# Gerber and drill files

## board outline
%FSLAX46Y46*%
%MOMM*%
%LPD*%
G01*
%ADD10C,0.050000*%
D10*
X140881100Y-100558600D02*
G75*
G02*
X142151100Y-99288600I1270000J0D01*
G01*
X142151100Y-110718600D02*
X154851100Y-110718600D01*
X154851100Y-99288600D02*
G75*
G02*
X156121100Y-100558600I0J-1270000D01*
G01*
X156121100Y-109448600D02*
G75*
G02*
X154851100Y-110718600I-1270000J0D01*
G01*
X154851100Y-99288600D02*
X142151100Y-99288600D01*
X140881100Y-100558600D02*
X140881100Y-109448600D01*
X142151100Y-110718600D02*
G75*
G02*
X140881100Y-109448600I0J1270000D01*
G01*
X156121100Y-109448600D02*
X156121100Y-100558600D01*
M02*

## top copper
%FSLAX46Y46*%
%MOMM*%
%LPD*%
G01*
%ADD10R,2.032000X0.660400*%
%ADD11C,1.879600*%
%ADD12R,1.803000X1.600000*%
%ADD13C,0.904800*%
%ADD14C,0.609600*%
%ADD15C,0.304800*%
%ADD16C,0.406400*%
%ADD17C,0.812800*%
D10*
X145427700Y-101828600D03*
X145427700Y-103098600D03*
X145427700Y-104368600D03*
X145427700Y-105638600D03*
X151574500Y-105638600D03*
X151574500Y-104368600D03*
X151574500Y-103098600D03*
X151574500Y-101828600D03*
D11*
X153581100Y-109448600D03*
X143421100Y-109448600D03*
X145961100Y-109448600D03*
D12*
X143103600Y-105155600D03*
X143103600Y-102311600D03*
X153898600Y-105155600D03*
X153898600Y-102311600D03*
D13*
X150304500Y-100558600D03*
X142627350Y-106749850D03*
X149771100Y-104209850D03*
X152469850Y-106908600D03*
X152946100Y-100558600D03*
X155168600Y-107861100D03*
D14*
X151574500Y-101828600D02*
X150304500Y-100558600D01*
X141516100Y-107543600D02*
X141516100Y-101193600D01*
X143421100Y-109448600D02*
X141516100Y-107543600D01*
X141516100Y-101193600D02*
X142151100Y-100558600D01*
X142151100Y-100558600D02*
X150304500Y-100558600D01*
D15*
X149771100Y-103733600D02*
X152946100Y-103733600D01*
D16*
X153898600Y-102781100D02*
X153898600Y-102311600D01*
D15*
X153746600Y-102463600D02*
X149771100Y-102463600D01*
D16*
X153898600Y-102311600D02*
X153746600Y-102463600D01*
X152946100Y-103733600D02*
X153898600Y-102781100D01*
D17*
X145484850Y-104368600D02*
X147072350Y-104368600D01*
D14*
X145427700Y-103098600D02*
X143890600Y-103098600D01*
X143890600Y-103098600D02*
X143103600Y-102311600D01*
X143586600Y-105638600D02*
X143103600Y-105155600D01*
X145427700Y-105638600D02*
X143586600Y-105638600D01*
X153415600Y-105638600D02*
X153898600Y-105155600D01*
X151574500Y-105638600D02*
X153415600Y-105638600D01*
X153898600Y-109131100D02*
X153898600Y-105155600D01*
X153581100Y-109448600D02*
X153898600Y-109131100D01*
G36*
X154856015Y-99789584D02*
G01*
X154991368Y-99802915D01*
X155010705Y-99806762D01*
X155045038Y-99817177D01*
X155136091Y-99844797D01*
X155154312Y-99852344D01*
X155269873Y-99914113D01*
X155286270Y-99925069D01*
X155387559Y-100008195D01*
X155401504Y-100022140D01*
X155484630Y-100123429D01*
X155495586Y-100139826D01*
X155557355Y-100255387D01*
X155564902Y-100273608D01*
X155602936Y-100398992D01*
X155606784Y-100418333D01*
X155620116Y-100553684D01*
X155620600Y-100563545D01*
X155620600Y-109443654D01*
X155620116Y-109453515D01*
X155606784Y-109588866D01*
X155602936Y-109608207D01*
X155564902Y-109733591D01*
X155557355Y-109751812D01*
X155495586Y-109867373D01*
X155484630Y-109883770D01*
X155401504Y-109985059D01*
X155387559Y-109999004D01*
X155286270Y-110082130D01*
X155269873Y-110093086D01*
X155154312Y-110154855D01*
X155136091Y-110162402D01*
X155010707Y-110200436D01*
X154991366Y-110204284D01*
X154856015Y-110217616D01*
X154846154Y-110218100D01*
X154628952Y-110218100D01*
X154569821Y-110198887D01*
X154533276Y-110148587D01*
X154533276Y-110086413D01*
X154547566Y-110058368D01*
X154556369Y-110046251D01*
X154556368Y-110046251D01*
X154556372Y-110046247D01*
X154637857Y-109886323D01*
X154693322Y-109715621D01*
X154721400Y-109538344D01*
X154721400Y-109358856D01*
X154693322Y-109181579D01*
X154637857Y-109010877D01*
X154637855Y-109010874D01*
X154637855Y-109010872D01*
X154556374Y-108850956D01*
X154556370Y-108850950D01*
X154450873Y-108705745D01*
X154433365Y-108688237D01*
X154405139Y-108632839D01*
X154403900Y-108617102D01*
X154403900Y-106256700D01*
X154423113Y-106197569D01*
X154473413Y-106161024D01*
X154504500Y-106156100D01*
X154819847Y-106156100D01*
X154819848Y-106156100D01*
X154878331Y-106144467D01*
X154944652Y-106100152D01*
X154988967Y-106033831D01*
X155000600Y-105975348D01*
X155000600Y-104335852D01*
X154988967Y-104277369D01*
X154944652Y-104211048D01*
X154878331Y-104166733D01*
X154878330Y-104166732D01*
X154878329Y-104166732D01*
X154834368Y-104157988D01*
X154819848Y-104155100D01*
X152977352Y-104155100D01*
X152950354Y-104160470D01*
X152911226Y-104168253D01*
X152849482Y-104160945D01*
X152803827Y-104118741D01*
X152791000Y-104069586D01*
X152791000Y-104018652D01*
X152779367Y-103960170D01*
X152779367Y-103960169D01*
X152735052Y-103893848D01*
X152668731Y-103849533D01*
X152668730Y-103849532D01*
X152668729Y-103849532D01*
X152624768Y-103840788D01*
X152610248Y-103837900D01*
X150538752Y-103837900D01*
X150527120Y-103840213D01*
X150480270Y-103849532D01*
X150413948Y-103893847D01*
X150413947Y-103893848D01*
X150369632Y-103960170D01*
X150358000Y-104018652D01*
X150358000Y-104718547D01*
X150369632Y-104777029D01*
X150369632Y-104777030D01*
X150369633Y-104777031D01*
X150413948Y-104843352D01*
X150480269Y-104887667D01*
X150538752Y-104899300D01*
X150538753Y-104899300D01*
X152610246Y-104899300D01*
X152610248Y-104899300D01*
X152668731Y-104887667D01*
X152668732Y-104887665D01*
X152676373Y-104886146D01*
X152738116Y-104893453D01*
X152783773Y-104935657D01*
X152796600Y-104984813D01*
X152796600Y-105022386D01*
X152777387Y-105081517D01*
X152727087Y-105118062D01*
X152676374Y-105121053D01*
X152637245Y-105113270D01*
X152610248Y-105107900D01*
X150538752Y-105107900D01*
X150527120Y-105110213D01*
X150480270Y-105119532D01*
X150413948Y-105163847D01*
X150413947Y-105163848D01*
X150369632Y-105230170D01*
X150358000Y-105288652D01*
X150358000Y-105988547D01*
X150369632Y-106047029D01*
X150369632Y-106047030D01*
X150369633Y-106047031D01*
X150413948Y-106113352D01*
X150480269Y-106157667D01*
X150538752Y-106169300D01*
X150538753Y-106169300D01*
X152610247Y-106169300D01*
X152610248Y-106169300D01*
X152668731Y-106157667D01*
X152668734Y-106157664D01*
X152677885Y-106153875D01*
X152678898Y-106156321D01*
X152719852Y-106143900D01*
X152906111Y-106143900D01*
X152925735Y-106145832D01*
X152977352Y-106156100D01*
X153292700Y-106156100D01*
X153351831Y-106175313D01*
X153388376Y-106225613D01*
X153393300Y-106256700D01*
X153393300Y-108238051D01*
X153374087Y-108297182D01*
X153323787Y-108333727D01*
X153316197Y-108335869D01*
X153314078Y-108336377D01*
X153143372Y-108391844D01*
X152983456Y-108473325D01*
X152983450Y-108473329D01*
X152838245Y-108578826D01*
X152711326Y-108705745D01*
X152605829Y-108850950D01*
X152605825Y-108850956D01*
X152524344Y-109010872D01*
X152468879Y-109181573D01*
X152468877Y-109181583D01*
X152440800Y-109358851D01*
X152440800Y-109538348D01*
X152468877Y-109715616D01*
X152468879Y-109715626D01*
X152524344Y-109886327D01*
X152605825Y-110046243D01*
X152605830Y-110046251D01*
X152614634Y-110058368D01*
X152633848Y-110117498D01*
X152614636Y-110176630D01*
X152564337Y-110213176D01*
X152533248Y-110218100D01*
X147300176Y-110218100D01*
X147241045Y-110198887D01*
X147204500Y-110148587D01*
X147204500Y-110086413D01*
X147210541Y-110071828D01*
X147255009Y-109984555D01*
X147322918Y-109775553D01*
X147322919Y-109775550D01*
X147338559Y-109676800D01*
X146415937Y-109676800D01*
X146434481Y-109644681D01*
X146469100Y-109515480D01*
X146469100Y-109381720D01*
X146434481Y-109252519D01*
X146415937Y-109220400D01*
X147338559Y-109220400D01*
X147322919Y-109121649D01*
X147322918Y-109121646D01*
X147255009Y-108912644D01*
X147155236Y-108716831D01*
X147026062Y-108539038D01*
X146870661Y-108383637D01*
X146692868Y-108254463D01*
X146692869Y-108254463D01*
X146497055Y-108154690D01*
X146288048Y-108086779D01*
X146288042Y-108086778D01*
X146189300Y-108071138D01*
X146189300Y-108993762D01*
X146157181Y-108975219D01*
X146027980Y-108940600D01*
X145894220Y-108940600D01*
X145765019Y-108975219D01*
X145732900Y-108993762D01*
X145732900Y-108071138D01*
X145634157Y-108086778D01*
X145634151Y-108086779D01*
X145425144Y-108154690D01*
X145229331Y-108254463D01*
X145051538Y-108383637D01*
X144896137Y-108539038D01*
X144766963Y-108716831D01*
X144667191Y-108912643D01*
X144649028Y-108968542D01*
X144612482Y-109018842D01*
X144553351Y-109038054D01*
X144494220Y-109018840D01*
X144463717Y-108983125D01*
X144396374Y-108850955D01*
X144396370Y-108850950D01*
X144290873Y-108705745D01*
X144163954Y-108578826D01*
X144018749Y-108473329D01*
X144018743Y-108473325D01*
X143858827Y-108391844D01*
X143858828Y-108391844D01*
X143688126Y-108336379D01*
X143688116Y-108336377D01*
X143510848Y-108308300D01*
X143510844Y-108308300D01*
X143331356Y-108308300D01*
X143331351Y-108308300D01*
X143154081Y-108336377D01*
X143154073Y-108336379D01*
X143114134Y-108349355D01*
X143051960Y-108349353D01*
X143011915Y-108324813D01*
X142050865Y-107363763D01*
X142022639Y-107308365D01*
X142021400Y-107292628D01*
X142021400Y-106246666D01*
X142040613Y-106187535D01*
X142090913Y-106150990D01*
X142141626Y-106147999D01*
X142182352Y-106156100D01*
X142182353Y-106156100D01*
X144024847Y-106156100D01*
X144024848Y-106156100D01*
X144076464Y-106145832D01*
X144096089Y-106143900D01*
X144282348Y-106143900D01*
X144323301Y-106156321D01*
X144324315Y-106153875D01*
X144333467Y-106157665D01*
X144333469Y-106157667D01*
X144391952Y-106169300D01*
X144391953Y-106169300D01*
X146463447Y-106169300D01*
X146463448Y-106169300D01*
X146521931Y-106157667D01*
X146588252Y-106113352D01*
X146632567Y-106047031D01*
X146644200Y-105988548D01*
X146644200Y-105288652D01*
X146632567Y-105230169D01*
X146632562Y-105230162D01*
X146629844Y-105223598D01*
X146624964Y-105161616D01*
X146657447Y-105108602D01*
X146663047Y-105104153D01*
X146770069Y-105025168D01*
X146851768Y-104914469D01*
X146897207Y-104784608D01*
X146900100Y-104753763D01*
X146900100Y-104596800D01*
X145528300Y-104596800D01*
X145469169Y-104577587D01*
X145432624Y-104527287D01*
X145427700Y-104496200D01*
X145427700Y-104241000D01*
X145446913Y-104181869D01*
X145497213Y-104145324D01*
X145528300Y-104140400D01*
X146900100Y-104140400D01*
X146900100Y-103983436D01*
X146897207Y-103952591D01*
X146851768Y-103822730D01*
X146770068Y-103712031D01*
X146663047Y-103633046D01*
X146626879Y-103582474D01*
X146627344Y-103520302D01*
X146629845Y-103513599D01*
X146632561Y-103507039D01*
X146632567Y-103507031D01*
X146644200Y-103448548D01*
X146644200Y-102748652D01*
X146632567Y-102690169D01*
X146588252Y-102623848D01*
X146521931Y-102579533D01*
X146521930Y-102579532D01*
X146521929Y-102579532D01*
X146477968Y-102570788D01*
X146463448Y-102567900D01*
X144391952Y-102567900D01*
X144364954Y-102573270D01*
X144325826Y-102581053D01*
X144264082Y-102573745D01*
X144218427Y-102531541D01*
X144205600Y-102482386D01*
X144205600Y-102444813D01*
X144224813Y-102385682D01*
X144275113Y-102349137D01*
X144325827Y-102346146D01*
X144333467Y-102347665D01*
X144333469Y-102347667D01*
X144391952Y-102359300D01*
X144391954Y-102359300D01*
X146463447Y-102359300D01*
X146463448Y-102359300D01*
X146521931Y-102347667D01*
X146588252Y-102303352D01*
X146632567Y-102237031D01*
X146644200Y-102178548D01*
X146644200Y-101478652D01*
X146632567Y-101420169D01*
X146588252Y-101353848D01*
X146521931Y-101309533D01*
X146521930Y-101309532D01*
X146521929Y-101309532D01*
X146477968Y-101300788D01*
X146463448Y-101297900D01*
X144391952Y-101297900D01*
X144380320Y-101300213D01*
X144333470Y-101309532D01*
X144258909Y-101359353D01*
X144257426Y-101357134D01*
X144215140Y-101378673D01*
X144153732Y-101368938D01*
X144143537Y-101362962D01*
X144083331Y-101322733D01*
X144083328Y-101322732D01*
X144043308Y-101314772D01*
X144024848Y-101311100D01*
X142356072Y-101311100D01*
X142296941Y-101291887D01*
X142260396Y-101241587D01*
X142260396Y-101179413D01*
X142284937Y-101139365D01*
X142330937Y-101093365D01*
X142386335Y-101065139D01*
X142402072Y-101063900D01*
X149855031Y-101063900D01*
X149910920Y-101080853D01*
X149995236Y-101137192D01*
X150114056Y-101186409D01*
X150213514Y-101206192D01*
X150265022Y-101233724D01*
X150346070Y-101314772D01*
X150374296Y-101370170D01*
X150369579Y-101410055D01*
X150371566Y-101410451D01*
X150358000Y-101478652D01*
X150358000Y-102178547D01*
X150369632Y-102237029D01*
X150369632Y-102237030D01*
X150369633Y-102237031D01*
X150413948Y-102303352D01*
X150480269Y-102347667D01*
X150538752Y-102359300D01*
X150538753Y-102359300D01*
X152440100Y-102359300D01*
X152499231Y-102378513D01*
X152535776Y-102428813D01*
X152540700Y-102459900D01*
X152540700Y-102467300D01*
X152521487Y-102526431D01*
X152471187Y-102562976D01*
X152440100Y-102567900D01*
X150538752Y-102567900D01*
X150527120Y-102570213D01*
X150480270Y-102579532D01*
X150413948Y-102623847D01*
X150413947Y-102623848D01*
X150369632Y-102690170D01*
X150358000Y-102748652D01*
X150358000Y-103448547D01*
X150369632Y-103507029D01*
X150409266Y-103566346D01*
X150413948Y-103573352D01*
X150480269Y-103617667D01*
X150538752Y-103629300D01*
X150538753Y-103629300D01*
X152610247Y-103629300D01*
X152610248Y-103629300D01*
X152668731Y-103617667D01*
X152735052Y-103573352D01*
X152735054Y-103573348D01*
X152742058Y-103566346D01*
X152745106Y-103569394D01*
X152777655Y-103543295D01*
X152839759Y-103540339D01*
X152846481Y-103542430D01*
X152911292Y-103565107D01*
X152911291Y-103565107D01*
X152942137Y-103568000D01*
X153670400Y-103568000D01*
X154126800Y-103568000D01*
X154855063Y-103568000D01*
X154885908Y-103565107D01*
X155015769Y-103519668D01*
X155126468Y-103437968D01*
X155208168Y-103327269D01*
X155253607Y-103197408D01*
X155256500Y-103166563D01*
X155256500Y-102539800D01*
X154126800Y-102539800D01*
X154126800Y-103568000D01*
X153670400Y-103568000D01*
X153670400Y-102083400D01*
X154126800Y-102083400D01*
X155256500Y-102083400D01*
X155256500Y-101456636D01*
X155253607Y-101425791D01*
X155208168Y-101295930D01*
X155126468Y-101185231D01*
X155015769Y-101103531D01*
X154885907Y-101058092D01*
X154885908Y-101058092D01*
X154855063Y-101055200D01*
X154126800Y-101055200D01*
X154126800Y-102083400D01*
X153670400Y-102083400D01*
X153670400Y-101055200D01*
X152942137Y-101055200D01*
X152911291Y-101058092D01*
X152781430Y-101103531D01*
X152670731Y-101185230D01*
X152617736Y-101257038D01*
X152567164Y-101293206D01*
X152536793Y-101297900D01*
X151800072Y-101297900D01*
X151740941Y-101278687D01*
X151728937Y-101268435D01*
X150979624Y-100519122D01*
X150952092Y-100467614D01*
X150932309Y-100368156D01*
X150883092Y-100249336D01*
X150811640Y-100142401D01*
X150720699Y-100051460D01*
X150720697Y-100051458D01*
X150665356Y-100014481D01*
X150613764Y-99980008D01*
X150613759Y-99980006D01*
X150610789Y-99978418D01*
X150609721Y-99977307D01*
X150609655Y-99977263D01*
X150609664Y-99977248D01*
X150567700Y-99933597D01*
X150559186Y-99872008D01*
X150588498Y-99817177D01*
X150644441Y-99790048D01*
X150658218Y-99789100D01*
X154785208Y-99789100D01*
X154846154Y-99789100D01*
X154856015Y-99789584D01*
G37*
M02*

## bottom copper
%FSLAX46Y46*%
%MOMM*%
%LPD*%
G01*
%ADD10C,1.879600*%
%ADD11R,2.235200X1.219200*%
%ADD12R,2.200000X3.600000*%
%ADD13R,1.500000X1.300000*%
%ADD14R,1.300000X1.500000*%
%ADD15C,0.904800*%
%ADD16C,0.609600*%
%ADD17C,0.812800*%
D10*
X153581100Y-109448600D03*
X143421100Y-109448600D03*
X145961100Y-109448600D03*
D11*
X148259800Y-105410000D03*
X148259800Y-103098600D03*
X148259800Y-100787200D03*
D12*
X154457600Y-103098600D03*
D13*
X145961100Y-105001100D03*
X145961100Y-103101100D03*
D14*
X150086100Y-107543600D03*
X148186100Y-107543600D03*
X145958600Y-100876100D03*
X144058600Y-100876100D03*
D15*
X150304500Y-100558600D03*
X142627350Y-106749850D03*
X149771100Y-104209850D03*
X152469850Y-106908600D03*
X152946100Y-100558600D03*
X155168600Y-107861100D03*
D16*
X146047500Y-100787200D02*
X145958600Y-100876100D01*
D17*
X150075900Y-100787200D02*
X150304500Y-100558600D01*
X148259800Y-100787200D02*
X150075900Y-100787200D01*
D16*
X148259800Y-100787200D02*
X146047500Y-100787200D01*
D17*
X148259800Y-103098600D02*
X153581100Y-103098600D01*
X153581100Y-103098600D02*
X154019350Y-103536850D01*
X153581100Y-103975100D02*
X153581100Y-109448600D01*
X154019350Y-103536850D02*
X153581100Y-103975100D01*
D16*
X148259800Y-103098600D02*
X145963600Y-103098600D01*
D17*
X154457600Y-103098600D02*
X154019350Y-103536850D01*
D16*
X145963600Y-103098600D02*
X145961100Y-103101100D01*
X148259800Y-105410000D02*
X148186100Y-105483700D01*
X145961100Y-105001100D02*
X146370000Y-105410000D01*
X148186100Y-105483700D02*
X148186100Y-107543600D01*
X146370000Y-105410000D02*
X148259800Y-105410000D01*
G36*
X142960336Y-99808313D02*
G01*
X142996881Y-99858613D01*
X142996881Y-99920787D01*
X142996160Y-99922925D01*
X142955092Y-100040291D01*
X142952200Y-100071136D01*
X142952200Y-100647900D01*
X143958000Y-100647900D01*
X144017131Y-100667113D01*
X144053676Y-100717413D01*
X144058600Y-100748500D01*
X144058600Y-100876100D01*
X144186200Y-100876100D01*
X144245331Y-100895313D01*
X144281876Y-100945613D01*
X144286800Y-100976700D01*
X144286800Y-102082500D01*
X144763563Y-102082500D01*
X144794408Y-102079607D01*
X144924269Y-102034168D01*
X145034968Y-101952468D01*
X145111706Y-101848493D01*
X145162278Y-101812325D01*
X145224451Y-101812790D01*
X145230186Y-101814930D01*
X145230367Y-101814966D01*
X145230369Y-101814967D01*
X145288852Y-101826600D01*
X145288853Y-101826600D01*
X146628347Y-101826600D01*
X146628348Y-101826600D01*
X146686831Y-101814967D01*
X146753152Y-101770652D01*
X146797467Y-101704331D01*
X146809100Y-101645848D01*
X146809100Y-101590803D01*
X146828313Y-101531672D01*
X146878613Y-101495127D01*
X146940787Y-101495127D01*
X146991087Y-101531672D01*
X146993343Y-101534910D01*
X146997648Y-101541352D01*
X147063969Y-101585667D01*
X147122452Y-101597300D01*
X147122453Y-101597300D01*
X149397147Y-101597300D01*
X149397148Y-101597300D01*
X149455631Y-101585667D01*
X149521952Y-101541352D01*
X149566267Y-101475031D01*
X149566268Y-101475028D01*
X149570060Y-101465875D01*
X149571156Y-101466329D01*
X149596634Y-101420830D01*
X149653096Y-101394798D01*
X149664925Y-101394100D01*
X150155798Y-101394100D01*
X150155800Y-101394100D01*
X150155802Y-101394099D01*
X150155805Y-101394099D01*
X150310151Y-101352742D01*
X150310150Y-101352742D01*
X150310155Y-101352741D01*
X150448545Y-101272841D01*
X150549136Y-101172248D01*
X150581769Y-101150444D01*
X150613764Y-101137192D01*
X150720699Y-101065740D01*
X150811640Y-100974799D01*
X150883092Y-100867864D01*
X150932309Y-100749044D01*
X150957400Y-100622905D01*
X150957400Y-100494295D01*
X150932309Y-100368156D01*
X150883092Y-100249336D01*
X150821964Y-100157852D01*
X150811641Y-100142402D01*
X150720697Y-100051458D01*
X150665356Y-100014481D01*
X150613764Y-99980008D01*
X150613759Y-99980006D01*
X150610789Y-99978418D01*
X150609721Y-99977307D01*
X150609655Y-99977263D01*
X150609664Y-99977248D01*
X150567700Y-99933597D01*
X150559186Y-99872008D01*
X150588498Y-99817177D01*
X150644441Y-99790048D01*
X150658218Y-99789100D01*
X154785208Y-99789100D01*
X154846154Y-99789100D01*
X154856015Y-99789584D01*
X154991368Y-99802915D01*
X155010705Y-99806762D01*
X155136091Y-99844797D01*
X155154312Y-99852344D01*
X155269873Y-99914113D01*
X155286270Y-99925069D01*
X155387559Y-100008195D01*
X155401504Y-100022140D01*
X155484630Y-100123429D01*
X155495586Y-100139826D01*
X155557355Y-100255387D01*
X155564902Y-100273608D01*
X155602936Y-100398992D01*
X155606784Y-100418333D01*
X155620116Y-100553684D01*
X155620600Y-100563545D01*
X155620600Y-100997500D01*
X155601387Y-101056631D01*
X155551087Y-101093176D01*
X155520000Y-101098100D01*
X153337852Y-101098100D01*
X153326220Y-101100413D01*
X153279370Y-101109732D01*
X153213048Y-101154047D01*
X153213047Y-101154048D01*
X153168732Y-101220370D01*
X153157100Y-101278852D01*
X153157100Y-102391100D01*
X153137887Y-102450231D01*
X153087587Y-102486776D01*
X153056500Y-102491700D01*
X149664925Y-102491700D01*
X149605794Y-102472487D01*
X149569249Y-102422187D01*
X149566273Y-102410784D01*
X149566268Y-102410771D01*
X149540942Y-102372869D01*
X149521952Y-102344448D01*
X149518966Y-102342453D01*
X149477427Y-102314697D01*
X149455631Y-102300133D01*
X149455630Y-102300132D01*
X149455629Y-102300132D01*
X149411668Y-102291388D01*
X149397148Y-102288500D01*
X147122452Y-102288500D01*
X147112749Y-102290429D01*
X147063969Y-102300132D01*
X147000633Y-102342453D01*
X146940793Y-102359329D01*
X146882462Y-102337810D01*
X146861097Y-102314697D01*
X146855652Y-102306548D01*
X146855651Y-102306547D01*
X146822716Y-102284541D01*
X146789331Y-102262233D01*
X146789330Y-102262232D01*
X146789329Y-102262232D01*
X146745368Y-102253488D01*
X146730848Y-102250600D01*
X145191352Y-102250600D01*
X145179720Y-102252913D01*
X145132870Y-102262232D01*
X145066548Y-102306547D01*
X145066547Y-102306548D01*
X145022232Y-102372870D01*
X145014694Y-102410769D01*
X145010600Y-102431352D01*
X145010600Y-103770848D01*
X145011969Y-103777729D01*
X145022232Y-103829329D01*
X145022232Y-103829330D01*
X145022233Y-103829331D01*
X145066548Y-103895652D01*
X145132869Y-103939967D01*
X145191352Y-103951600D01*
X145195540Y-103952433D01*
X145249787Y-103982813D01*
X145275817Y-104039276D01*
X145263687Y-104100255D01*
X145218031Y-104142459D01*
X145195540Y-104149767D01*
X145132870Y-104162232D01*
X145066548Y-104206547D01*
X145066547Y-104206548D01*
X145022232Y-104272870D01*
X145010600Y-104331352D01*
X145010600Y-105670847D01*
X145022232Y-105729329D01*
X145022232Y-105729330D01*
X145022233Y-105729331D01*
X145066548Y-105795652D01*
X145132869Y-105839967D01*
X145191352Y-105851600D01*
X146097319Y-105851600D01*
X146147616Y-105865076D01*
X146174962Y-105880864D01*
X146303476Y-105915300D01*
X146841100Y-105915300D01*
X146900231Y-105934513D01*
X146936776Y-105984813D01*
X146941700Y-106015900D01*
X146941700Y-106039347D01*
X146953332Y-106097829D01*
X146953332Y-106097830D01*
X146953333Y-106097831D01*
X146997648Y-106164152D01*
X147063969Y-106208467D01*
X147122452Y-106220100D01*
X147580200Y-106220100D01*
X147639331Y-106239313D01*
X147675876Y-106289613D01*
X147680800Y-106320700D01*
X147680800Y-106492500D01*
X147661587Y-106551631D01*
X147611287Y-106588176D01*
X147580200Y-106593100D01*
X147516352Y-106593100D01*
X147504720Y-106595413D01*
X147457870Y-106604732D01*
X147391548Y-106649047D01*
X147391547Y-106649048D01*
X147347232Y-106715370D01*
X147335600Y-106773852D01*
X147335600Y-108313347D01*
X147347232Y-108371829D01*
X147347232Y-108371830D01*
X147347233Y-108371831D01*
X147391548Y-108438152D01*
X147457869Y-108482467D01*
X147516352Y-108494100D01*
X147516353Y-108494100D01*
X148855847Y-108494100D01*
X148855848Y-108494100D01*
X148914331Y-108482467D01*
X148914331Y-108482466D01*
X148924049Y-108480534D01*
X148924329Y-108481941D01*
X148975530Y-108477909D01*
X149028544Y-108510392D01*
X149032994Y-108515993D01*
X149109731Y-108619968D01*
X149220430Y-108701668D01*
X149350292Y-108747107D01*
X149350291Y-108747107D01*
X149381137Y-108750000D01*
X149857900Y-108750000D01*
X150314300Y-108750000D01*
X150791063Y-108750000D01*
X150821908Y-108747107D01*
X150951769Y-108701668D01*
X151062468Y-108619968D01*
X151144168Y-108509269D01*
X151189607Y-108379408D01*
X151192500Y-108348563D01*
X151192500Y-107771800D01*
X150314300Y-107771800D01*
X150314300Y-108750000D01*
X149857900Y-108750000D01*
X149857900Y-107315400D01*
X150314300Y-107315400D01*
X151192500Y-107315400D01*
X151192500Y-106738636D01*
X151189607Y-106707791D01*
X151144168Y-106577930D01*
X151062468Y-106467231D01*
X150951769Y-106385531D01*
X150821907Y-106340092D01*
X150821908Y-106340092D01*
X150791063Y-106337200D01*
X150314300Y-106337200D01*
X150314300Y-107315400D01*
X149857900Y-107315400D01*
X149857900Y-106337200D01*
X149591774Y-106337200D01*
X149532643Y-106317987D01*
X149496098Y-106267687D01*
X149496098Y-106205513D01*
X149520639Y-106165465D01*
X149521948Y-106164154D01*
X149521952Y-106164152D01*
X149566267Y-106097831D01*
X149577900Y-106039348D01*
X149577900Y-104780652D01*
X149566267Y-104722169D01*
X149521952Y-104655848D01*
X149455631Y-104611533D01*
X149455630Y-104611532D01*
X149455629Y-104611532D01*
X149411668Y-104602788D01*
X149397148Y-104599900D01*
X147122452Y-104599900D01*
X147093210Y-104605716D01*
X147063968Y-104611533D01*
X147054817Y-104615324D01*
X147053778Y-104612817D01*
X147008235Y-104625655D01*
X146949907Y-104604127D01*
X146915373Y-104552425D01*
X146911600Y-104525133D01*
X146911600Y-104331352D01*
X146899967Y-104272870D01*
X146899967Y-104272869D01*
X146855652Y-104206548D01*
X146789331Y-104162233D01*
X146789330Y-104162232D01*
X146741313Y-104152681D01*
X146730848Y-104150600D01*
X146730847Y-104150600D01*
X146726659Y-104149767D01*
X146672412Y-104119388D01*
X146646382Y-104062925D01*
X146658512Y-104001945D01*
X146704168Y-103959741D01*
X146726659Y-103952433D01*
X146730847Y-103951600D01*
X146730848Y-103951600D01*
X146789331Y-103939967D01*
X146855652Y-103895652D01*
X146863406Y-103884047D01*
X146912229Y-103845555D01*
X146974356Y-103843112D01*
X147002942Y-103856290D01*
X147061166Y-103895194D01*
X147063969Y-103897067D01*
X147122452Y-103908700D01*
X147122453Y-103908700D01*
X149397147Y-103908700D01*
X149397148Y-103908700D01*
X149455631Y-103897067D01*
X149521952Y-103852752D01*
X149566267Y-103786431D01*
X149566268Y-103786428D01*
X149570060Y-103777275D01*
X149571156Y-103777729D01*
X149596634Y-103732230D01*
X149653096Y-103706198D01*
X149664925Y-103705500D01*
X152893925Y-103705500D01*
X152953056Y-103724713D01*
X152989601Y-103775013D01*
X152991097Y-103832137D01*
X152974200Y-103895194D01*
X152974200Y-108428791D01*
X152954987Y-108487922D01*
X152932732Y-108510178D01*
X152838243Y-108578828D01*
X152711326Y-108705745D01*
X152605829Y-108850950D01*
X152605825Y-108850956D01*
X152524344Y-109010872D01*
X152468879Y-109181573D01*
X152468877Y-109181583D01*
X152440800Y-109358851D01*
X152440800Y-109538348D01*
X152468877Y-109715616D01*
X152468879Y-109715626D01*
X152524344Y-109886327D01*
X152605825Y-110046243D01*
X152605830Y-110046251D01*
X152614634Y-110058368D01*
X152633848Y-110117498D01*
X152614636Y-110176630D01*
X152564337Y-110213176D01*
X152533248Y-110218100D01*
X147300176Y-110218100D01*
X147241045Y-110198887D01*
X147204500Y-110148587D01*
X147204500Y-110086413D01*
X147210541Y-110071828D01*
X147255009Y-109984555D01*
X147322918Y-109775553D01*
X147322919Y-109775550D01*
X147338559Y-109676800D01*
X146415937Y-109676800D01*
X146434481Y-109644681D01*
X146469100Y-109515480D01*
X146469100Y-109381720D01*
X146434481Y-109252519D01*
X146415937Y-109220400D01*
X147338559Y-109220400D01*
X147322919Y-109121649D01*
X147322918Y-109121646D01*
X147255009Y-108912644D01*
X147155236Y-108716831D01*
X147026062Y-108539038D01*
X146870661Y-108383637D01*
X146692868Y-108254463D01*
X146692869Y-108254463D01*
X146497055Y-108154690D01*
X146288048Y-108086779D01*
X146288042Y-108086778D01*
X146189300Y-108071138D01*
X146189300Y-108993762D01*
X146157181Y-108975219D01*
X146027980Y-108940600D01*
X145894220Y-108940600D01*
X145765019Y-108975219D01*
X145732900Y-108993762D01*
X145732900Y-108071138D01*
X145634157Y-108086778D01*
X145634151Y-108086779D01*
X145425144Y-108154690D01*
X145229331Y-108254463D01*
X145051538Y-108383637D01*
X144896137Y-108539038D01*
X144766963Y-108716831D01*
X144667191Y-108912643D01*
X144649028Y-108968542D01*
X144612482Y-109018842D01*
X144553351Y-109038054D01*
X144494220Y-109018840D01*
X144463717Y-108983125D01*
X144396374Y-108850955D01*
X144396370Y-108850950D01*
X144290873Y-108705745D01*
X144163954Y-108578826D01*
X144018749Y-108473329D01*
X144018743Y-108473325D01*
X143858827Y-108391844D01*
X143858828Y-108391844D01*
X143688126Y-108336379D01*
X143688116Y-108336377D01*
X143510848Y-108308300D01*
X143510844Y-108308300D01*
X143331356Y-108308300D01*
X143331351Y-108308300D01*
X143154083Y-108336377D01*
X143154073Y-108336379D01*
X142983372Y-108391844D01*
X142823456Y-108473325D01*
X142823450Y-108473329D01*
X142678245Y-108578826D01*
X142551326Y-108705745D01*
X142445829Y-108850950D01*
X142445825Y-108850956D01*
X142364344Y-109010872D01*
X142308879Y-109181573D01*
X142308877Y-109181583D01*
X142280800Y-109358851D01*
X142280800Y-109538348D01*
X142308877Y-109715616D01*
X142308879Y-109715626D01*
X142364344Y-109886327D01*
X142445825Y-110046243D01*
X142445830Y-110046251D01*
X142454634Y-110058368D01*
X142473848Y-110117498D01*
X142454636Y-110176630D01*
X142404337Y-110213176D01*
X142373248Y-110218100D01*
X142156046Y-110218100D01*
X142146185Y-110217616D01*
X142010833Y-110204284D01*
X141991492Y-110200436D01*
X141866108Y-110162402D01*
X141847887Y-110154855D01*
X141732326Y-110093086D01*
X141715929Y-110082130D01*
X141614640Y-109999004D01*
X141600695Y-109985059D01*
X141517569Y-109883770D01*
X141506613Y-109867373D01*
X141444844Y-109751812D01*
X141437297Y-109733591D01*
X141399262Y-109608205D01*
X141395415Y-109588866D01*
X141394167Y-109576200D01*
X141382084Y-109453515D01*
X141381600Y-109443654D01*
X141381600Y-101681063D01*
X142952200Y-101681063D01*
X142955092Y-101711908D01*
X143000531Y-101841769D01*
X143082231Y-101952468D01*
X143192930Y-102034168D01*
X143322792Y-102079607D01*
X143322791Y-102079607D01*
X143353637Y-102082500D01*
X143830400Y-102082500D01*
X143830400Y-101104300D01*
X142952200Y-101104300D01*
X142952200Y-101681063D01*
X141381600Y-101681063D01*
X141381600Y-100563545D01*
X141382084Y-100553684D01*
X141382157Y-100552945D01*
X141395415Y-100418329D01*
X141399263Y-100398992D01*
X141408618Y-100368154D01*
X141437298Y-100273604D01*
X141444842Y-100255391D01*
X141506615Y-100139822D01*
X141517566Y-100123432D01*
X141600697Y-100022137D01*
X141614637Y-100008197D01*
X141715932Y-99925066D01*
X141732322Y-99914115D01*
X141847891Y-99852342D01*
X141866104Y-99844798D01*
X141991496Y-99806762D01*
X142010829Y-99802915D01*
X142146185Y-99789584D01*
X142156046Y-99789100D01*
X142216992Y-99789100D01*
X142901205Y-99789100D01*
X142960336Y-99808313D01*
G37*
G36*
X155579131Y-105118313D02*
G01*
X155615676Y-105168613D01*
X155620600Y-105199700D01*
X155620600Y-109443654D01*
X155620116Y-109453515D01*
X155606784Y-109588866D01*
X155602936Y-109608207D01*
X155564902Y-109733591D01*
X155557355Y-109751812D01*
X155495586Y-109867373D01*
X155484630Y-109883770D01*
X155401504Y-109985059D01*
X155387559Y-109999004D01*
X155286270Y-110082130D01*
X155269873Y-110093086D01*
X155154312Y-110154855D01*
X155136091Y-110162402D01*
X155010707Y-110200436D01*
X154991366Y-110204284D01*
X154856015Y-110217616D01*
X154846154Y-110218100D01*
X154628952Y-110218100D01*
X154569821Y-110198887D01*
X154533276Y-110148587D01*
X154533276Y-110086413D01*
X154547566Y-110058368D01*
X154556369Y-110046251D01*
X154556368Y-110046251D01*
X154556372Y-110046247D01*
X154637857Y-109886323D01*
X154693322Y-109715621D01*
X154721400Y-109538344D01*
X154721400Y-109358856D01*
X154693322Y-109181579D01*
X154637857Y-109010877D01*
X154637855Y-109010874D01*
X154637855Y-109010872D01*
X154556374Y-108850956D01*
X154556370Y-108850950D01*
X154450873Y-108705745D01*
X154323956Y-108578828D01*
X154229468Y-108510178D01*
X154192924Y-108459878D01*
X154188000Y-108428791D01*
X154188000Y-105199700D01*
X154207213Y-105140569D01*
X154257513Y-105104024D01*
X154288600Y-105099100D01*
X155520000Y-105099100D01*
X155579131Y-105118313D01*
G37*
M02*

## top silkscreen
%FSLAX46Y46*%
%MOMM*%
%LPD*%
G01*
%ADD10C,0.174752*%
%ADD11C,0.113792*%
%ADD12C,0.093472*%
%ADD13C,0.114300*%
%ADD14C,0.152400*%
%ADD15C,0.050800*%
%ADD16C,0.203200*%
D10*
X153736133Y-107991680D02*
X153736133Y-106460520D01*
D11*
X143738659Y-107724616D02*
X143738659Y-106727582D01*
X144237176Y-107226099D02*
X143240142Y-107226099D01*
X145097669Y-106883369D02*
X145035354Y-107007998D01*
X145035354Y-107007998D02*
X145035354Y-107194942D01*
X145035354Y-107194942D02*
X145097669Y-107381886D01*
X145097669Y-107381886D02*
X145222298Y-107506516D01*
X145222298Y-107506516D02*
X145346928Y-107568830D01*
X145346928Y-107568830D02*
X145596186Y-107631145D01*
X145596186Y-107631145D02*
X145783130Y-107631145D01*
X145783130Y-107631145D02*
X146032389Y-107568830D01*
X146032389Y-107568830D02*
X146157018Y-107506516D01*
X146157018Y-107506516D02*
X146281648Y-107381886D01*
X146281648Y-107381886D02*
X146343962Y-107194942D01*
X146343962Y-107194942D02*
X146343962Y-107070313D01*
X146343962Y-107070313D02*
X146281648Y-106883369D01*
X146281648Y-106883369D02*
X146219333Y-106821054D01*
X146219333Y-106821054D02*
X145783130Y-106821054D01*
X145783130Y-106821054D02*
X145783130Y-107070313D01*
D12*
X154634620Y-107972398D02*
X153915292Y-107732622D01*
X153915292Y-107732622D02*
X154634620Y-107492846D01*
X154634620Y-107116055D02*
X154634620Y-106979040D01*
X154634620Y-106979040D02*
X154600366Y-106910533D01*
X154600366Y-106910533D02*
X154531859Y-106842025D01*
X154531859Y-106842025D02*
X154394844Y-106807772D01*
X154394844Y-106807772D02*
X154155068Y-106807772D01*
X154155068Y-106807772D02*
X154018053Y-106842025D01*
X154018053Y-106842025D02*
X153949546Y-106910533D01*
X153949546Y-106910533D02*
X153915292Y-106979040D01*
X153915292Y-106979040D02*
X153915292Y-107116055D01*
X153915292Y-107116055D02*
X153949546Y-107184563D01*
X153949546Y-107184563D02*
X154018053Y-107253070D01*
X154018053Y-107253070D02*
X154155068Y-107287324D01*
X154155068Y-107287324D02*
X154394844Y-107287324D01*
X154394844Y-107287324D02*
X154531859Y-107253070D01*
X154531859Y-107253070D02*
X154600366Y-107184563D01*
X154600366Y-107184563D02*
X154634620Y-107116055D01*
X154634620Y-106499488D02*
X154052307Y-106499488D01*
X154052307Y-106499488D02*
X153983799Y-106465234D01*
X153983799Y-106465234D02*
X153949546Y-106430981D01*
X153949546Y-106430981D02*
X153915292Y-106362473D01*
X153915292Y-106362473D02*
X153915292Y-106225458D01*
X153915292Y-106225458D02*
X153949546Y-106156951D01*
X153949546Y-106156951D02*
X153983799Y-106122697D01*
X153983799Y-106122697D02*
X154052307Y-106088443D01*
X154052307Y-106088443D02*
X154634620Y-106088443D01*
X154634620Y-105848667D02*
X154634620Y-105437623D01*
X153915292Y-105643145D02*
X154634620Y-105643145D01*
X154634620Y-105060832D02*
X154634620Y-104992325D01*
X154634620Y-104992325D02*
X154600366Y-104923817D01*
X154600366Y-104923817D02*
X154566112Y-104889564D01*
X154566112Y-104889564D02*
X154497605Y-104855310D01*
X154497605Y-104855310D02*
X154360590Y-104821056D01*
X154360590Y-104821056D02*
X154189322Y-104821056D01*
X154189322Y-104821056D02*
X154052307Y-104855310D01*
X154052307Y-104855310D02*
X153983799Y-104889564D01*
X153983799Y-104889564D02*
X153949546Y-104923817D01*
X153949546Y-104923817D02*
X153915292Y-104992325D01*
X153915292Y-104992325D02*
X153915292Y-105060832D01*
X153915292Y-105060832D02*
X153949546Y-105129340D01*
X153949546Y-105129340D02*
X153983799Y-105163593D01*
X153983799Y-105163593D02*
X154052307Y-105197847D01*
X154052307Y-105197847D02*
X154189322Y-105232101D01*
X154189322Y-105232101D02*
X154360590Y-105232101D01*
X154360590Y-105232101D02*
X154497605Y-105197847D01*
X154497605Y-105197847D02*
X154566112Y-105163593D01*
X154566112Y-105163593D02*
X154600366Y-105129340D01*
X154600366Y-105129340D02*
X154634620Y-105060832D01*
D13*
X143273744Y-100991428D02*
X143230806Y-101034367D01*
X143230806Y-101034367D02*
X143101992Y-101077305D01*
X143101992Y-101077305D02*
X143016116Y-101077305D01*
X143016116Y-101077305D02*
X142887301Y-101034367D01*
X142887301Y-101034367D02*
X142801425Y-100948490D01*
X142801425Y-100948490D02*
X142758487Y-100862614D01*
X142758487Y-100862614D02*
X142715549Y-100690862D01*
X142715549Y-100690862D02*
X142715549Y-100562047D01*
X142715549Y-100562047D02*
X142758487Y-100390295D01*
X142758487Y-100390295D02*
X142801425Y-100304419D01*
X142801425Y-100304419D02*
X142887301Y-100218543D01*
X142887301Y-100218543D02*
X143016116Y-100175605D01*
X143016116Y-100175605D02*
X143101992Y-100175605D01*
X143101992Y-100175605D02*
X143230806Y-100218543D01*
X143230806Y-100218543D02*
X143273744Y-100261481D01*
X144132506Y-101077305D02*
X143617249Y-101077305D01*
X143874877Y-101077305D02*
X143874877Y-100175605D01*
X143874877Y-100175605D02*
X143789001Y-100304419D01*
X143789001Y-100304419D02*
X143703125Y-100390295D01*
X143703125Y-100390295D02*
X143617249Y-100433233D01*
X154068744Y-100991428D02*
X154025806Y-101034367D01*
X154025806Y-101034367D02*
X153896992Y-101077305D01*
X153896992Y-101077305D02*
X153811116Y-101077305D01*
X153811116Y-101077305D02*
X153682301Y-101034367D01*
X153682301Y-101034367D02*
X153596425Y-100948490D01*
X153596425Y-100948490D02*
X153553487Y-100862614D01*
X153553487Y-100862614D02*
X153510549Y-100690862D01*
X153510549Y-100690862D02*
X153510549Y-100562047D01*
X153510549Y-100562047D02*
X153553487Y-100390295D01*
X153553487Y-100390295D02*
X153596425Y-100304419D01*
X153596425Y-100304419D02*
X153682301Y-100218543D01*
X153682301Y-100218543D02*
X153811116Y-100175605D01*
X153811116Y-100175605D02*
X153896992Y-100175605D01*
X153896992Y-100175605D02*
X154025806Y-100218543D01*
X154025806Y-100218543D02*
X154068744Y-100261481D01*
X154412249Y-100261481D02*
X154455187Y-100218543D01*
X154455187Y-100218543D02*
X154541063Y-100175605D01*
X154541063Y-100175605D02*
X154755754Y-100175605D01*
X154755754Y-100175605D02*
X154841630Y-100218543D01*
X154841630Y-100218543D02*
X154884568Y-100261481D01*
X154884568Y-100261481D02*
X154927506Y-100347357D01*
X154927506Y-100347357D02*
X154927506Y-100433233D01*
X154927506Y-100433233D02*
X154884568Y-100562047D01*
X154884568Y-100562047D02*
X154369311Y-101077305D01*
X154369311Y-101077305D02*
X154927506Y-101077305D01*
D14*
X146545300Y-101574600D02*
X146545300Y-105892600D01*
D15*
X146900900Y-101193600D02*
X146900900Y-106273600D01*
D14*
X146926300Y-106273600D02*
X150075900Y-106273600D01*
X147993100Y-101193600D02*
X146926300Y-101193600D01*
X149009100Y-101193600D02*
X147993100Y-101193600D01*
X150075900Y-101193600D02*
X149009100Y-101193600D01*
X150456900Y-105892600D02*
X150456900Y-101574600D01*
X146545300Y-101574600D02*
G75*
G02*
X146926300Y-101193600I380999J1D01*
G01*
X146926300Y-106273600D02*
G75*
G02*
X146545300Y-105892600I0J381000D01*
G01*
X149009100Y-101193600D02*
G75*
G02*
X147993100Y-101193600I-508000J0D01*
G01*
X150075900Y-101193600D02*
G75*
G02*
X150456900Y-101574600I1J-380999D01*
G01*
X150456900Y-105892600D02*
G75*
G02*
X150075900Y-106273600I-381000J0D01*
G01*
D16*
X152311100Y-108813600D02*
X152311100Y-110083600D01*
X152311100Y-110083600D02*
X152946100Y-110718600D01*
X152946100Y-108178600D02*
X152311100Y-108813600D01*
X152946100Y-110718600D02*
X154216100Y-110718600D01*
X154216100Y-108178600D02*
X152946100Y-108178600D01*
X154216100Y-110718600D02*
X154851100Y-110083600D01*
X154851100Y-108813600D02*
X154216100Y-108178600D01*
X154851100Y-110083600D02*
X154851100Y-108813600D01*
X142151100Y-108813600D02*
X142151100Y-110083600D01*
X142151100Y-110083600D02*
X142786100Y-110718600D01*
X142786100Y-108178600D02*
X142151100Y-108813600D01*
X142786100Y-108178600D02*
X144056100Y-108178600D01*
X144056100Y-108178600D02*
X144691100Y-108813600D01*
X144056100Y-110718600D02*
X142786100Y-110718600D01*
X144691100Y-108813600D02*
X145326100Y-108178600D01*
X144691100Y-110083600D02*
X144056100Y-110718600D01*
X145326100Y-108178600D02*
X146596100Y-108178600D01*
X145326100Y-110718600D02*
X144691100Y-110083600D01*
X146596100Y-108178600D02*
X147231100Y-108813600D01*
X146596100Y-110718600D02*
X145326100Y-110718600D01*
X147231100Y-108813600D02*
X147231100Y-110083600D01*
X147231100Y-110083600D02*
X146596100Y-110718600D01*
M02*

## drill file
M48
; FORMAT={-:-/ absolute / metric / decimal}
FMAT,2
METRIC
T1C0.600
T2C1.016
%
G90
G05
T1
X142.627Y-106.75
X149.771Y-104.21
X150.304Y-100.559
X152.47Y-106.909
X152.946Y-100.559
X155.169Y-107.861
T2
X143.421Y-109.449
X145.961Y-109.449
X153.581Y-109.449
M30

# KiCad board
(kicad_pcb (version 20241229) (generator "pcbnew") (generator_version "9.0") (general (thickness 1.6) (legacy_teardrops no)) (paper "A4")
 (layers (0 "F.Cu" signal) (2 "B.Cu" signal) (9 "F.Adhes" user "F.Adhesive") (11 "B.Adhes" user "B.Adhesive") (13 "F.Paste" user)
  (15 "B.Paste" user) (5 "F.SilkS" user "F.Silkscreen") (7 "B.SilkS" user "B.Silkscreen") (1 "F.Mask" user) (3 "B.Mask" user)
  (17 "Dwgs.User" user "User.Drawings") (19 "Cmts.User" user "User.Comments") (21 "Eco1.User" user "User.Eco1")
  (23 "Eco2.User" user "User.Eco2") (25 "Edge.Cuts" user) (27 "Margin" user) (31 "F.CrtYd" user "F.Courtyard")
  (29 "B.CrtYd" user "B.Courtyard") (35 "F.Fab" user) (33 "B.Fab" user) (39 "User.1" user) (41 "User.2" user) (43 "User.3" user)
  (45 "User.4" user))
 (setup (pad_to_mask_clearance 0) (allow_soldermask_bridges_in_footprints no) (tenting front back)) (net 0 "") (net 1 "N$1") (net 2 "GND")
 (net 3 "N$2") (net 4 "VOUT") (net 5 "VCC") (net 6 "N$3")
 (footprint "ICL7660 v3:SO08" (layer "F.Cu") (at 148.5011 103.7336 -90)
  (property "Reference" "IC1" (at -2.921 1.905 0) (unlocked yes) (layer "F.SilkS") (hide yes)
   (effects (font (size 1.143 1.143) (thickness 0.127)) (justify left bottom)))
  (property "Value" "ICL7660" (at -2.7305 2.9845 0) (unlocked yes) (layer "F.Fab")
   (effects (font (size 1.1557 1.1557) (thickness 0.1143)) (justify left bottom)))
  (fp_line (start -2.159 1.9558) (end 2.159 1.9558) (stroke (width 0.1524) (type solid)) (layer "F.SilkS"))
  (fp_line (start -2.54 1.6002) (end 2.54 1.6002) (stroke (width 0.0508) (type solid)) (layer "F.SilkS"))
  (fp_line (start 2.54 1.5748) (end 2.54 -1.5748) (stroke (width 0.1524) (type solid)) (layer "F.SilkS"))
  (fp_line (start -2.54 0.508) (end -2.54 1.5748) (stroke (width 0.1524) (type solid)) (layer "F.SilkS"))
  (fp_line (start -2.54 -0.508) (end -2.54 0.508) (stroke (width 0.1524) (type solid)) (layer "F.SilkS"))
  (fp_line (start -2.54 -1.5748) (end -2.54 -0.508) (stroke (width 0.1524) (type solid)) (layer "F.SilkS"))
  (fp_line (start 2.159 -1.9558) (end -2.159 -1.9558) (stroke (width 0.1524) (type solid)) (layer "F.SilkS"))
  (fp_arc (start -2.159 1.9558) (mid -2.428408 1.844208) (end -2.54 1.5748) (stroke (width 0.1524) (type solid)) (layer "F.SilkS"))
  (fp_arc (start 2.54 1.5748) (mid 2.428408 1.844208) (end 2.159 1.9558) (stroke (width 0.1524) (type solid)) (layer "F.SilkS"))
  (fp_arc (start -2.54 -0.508) (mid -2.032 0) (end -2.54 0.508) (stroke (width 0.1524) (type solid)) (layer "F.SilkS"))
  (fp_arc (start -2.54 -1.5748) (mid -2.428408 -1.844208) (end -2.159 -1.9558) (stroke (width 0.1524) (type solid)) (layer "F.SilkS"))
  (fp_arc (start 2.159 -1.9558) (mid 2.428408 -1.844208) (end 2.54 -1.5748) (stroke (width 0.1524) (type solid)) (layer "F.SilkS"))
  (pad "1" smd rect (at -1.905 3.0734 270) (size 0.6604 2.032) (layers "F.Cu" "F.Mask" "F.Paste") (solder_mask_margin 0.0508)
   (solder_paste_margin 0) (thermal_bridge_angle 0))
  (pad "2" smd rect (at -0.635 3.0734 270) (size 0.6604 2.032) (layers "F.Cu" "F.Mask" "F.Paste") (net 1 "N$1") (solder_mask_margin 0.0508)
   (solder_paste_margin 0) (thermal_bridge_angle 0))
  (pad "3" smd rect (at 0.635 3.0734 270) (size 0.6604 2.032) (layers "F.Cu" "F.Mask" "F.Paste") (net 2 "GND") (solder_mask_margin 0.0508)
   (solder_paste_margin 0) (thermal_bridge_angle 0))
  (pad "4" smd rect (at 1.905 3.0734 270) (size 0.6604 2.032) (layers "F.Cu" "F.Mask" "F.Paste") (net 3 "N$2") (solder_mask_margin 0.0508)
   (solder_paste_margin 0) (thermal_bridge_angle 0))
  (pad "5" smd rect (at 1.905 -3.0734 270) (size 0.6604 2.032) (layers "F.Cu" "F.Mask" "F.Paste") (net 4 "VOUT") (solder_mask_margin 0.0508)
   (solder_paste_margin 0) (thermal_bridge_angle 0))
  (pad "6" smd rect (at 0.635 -3.0734 270) (size 0.6604 2.032) (layers "F.Cu" "F.Mask" "F.Paste") (solder_mask_margin 0.0508)
   (solder_paste_margin 0) (thermal_bridge_angle 0))
  (pad "7" smd rect (at -0.635 -3.0734 270) (size 0.6604 2.032) (layers "F.Cu" "F.Mask" "F.Paste") (solder_mask_margin 0.0508)
   (solder_paste_margin 0) (thermal_bridge_angle 0))
  (pad "8" smd rect (at -1.905 -3.0734 270) (size 0.6604 2.032) (layers "F.Cu" "F.Mask" "F.Paste") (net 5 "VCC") (solder_mask_margin 0.0508)
   (solder_paste_margin 0) (thermal_bridge_angle 0)))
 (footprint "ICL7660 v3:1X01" (layer "F.Cu") (at 153.5811 109.4486)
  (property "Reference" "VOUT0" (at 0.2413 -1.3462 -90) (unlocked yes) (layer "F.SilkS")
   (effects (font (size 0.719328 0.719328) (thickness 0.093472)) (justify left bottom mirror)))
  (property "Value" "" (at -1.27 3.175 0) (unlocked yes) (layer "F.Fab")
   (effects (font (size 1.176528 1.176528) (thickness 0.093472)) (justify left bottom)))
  (fp_line (start -1.27 -0.635) (end -1.27 0.635) (stroke (width 0.2032) (type solid)) (layer "F.SilkS"))
  (fp_line (start -1.27 0.635) (end -0.635 1.27) (stroke (width 0.2032) (type solid)) (layer "F.SilkS"))
  (fp_line (start -0.635 -1.27) (end -1.27 -0.635) (stroke (width 0.2032) (type solid)) (layer "F.SilkS"))
  (fp_line (start -0.635 1.27) (end 0.635 1.27) (stroke (width 0.2032) (type solid)) (layer "F.SilkS"))
  (fp_line (start 0.635 -1.27) (end -0.635 -1.27) (stroke (width 0.2032) (type solid)) (layer "F.SilkS"))
  (fp_line (start 0.635 1.27) (end 1.27 0.635) (stroke (width 0.2032) (type solid)) (layer "F.SilkS"))
  (fp_line (start 1.27 -0.635) (end 0.635 -1.27) (stroke (width 0.2032) (type solid)) (layer "F.SilkS"))
  (fp_line (start 1.27 0.635) (end 1.27 -0.635) (stroke (width 0.2032) (type solid)) (layer "F.SilkS"))
  (pad "1" thru_hole circle (at 0 0 90) (size 1.8796 1.8796) (drill 1.016) (layers "*.Cu" "*.Mask") (remove_unused_layers no) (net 4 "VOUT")
   (solder_mask_margin 0.0508) (thermal_bridge_angle 0)))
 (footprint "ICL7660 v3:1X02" (layer "F.Cu") (at 143.4211 109.4486)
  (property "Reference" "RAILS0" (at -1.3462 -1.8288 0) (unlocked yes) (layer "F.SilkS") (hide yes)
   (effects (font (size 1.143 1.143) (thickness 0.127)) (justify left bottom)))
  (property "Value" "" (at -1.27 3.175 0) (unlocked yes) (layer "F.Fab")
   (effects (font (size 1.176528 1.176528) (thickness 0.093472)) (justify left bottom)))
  (fp_line (start -1.27 -0.635) (end -1.27 0.635) (stroke (width 0.2032) (type solid)) (layer "F.SilkS"))
  (fp_line (start -1.27 0.635) (end -0.635 1.27) (stroke (width 0.2032) (type solid)) (layer "F.SilkS"))
  (fp_line (start -0.635 -1.27) (end -1.27 -0.635) (stroke (width 0.2032) (type solid)) (layer "F.SilkS"))
  (fp_line (start -0.635 -1.27) (end 0.635 -1.27) (stroke (width 0.2032) (type solid)) (layer "F.SilkS"))
  (fp_line (start 0.635 -1.27) (end 1.27 -0.635) (stroke (width 0.2032) (type solid)) (layer "F.SilkS"))
  (fp_line (start 0.635 1.27) (end -0.635 1.27) (stroke (width 0.2032) (type solid)) (layer "F.SilkS"))
  (fp_line (start 1.27 -0.635) (end 1.905 -1.27) (stroke (width 0.2032) (type solid)) (layer "F.SilkS"))
  (fp_line (start 1.27 0.635) (end 0.635 1.27) (stroke (width 0.2032) (type solid)) (layer "F.SilkS"))
  (fp_line (start 1.905 -1.27) (end 3.175 -1.27) (stroke (width 0.2032) (type solid)) (layer "F.SilkS"))
  (fp_line (start 1.905 1.27) (end 1.27 0.635) (stroke (width 0.2032) (type solid)) (layer "F.SilkS"))
  (fp_line (start 3.175 -1.27) (end 3.81 -0.635) (stroke (width 0.2032) (type solid)) (layer "F.SilkS"))
  (fp_line (start 3.175 1.27) (end 1.905 1.27) (stroke (width 0.2032) (type solid)) (layer "F.SilkS"))
  (fp_line (start 3.81 -0.635) (end 3.81 0.635) (stroke (width 0.2032) (type solid)) (layer "F.SilkS"))
  (fp_line (start 3.81 0.635) (end 3.175 1.27) (stroke (width 0.2032) (type solid)) (layer "F.SilkS"))
  (pad "1" thru_hole circle (at 0 0 90) (size 1.8796 1.8796) (drill 1.016) (layers "*.Cu" "*.Mask") (remove_unused_layers no) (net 5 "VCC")
   (solder_mask_margin 0.0508) (thermal_bridge_angle 0))
  (pad "2" thru_hole circle (at 2.54 0 90) (size 1.8796 1.8796) (drill 1.016) (layers "*.Cu" "*.Mask") (remove_unused_layers no)
   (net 2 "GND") (solder_mask_margin 0.0508) (thermal_bridge_angle 0)))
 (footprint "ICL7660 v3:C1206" (layer "F.Cu") (at 143.1036 103.7336 90)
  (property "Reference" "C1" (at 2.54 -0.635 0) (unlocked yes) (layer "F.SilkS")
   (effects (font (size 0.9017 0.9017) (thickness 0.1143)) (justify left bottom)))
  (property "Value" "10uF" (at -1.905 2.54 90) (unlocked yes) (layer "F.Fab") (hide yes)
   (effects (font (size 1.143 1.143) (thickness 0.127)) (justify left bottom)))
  (pad "1" smd rect (at -1.422 0 90) (size 1.6 1.803) (layers "F.Cu" "F.Mask" "F.Paste") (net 3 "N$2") (solder_mask_margin 0.0508)
   (solder_paste_margin 0) (thermal_bridge_angle 0))
  (pad "2" smd rect (at 1.422 0 90) (size 1.6 1.803) (layers "F.Cu" "F.Mask" "F.Paste") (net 1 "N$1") (solder_mask_margin 0.0508)
   (solder_paste_margin 0) (thermal_bridge_angle 0)))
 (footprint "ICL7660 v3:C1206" (layer "F.Cu") (at 153.8986 103.7336 90)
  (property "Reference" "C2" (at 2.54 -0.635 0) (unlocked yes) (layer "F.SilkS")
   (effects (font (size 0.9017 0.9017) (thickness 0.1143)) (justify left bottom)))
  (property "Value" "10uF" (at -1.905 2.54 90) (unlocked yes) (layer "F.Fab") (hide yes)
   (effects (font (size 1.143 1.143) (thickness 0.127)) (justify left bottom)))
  (pad "1" smd rect (at -1.422 0 90) (size 1.6 1.803) (layers "F.Cu" "F.Mask" "F.Paste") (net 4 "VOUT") (solder_mask_margin 0.0508)
   (solder_paste_margin 0) (thermal_bridge_angle 0))
  (pad "2" smd rect (at 1.422 0 90) (size 1.6 1.803) (layers "F.Cu" "F.Mask" "F.Paste") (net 2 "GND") (solder_mask_margin 0.0508)
   (solder_paste_margin 0) (thermal_bridge_angle 0)))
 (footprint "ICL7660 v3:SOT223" (layer "B.Cu") (at 151.3586 103.0986 90)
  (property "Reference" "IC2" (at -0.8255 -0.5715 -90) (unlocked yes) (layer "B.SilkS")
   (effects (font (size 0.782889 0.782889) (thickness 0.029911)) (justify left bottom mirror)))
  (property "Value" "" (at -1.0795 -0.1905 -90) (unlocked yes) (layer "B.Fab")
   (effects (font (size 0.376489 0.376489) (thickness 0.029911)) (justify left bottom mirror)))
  (pad "1" smd rect (at -2.3114 -3.0988 90) (size 1.2192 2.2352) (layers "B.Cu" "B.Mask" "B.Paste") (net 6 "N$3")
   (solder_mask_margin 0.0508) (solder_paste_margin 0) (thermal_bridge_angle 0))
  (pad "2" smd rect (at 0 -3.0988 90) (size 1.2192 2.2352) (layers "B.Cu" "B.Mask" "B.Paste") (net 4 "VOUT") (solder_mask_margin 0.0508)
   (solder_paste_margin 0) (thermal_bridge_angle 0))
  (pad "3" smd rect (at 2.3114 -3.0988 90) (size 1.2192 2.2352) (layers "B.Cu" "B.Mask" "B.Paste") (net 5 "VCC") (solder_mask_margin 0.0508)
   (solder_paste_margin 0) (thermal_bridge_angle 0))
  (pad "4" smd rect (at 0 3.099 90) (size 3.6 2.2) (layers "B.Cu" "B.Mask" "B.Paste") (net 4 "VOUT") (solder_mask_margin 0.0508)
   (solder_paste_margin 0) (thermal_bridge_angle 0)))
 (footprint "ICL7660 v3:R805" (layer "B.Cu") (at 145.9611 104.0511 90)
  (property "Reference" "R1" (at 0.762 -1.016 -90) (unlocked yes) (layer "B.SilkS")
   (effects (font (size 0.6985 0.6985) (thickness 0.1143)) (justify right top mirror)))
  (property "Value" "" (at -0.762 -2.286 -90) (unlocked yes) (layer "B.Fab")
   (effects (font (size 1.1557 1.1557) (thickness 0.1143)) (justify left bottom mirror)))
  (pad "1" smd rect (at -0.95 0 90) (size 1.3 1.5) (layers "B.Cu" "B.Mask" "B.Paste") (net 6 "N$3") (solder_mask_margin 0.0508)
   (solder_paste_margin 0) (thermal_bridge_angle 0))
  (pad "2" smd rect (at 0.95 0 90) (size 1.3 1.5) (layers "B.Cu" "B.Mask" "B.Paste") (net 4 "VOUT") (solder_mask_margin 0.0508)
   (solder_paste_margin 0) (thermal_bridge_angle 0)))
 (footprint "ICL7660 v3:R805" (layer "B.Cu") (at 149.1361 107.5436 180)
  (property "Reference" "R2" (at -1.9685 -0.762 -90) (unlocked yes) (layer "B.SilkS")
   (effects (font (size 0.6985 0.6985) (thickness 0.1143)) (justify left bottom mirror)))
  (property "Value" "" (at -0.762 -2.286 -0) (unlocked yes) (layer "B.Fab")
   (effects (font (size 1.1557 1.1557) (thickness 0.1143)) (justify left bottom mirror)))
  (pad "1" smd rect (at -0.95 0 180) (size 1.3 1.5) (layers "B.Cu" "B.Mask" "B.Paste") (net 2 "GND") (solder_mask_margin 0.0508)
   (solder_paste_margin 0) (thermal_bridge_angle 0))
  (pad "2" smd rect (at 0.95 0 180) (size 1.3 1.5) (layers "B.Cu" "B.Mask" "B.Paste") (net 6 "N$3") (solder_mask_margin 0.0508)
   (solder_paste_margin 0) (thermal_bridge_angle 0)))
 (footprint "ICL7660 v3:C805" (layer "B.Cu") (at 145.0086 100.8761 180)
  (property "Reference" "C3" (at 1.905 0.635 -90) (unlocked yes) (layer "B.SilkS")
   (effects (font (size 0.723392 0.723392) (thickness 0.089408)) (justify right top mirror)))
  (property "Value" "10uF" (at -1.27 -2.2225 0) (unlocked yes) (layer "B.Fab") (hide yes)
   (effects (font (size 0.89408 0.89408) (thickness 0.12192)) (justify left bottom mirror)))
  (pad "1" smd rect (at -0.95 0 180) (size 1.3 1.5) (layers "B.Cu" "B.Mask" "B.Paste") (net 5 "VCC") (solder_mask_margin 0.0508)
   (solder_paste_margin 0) (thermal_bridge_angle 0))
  (pad "2" smd rect (at 0.95 0 180) (size 1.3 1.5) (layers "B.Cu" "B.Mask" "B.Paste") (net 2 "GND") (solder_mask_margin 0.0508)
   (solder_paste_margin 0) (thermal_bridge_angle 0)))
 (gr_arc (start 140.8811 100.5586) (mid 141.253074 99.660574) (end 142.1511 99.2886) (stroke (width 0.05) (type solid)) (layer "Edge.Cuts"))
 (gr_line (start 142.1511 110.7186) (end 154.8511 110.7186) (stroke (width 0.05) (type solid)) (layer "Edge.Cuts"))
 (gr_arc (start 154.8511 99.2886) (mid 155.749126 99.660574) (end 156.1211 100.5586) (stroke (width 0.05) (type solid)) (layer "Edge.Cuts"))
 (gr_arc (start 156.1211 109.4486) (mid 155.749126 110.346626) (end 154.8511 110.7186) (stroke (width 0.05) (type solid))
  (layer "Edge.Cuts"))
 (gr_line (start 154.8511 99.2886) (end 142.1511 99.2886) (stroke (width 0.05) (type solid)) (layer "Edge.Cuts"))
 (gr_line (start 140.8811 100.5586) (end 140.8811 109.4486) (stroke (width 0.05) (type solid)) (layer "Edge.Cuts"))
 (gr_arc (start 142.1511 110.7186) (mid 141.253074 110.346626) (end 140.8811 109.4486) (stroke (width 0.05) (type solid))
  (layer "Edge.Cuts"))
 (gr_line (start 156.1211 109.4486) (end 156.1211 100.5586) (stroke (width 0.05) (type solid)) (layer "Edge.Cuts"))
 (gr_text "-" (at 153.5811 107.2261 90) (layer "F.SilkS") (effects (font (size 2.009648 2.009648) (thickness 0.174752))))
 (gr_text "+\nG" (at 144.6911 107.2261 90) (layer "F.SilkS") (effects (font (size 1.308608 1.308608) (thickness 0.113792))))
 (segment (start 151.5745 101.8286) (end 150.3045 100.5586) (width 0.6096) (layer "F.Cu") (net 5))
 (segment (start 141.5161 107.5436) (end 141.5161 101.1936) (width 0.6096) (layer "F.Cu") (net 5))
 (segment (start 143.4211 109.4486) (end 141.5161 107.5436) (width 0.6096) (layer "F.Cu") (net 5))
 (segment (start 141.5161 101.1936) (end 142.1511 100.5586) (width 0.6096) (layer "F.Cu") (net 5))
 (segment (start 142.1511 100.5586) (end 150.3045 100.5586) (width 0.6096) (layer "F.Cu") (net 5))
 (via (at 150.3045 100.5586) (size 0.9048) (drill 0.6) (layers "F.Cu" "B.Cu") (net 5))
 (segment (start 146.0475 100.7872) (end 145.9586 100.8761) (width 0.6096) (layer "B.Cu") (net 5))
 (segment (start 150.0759 100.7872) (end 150.3045 100.5586) (width 0.8128) (layer "B.Cu") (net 5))
 (segment (start 148.2598 100.7872) (end 150.0759 100.7872) (width 0.8128) (layer "B.Cu") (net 5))
 (segment (start 148.2598 100.7872) (end 146.0475 100.7872) (width 0.6096) (layer "B.Cu") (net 5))
 (segment (start 149.7711 103.7336) (end 152.9461 103.7336) (width 0.3048) (layer "F.Cu") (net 2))
 (segment (start 153.8986 102.7811) (end 153.8986 102.3116) (width 0.4064) (layer "F.Cu") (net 2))
 (segment (start 153.7466 102.4636) (end 149.7711 102.4636) (width 0.3048) (layer "F.Cu") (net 2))
 (segment (start 153.8986 102.3116) (end 153.7466 102.4636) (width 0.4064) (layer "F.Cu") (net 2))
 (segment (start 152.9461 103.7336) (end 153.8986 102.7811) (width 0.4064) (layer "F.Cu") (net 2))
 (segment (start 145.48485 104.3686) (end 147.07235 104.3686) (width 0.8128) (layer "F.Cu") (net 2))
 (via (at 142.62735 106.74985) (size 0.9048) (drill 0.6) (layers "F.Cu" "B.Cu") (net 2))
 (via (at 149.7711 104.20985) (size 0.9048) (drill 0.6) (layers "F.Cu" "B.Cu") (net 2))
 (via (at 152.46985 106.9086) (size 0.9048) (drill 0.6) (layers "F.Cu" "B.Cu") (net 2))
 (via (at 152.9461 100.5586) (size 0.9048) (drill 0.6) (layers "F.Cu" "B.Cu") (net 2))
 (via (at 155.1686 107.8611) (size 0.9048) (drill 0.6) (layers "F.Cu" "B.Cu") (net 2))
 (segment (start 145.4277 103.0986) (end 143.8906 103.0986) (width 0.6096) (layer "F.Cu") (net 1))
 (segment (start 143.8906 103.0986) (end 143.1036 102.3116) (width 0.6096) (layer "F.Cu") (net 1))
 (segment (start 143.5866 105.6386) (end 143.1036 105.1556) (width 0.6096) (layer "F.Cu") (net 3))
 (segment (start 145.4277 105.6386) (end 143.5866 105.6386) (width 0.6096) (layer "F.Cu") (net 3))
 (segment (start 153.4156 105.6386) (end 153.8986 105.1556) (width 0.6096) (layer "F.Cu") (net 4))
 (segment (start 151.5745 105.6386) (end 153.4156 105.6386) (width 0.6096) (layer "F.Cu") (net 4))
 (segment (start 153.8986 109.1311) (end 153.8986 105.1556) (width 0.6096) (layer "F.Cu") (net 4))
 (segment (start 153.5811 109.4486) (end 153.8986 109.1311) (width 0.6096) (layer "F.Cu") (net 4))
 (segment (start 148.2598 103.0986) (end 153.5811 103.0986) (width 0.8128) (layer "B.Cu") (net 4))
 (segment (start 153.5811 103.0986) (end 154.01935 103.53685) (width 0.8128) (layer "B.Cu") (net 4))
 (segment (start 153.5811 103.9751) (end 153.5811 109.4486) (width 0.8128) (layer "B.Cu") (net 4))
 (segment (start 154.01935 103.53685) (end 153.5811 103.9751) (width 0.8128) (layer "B.Cu") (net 4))
 (segment (start 148.2598 103.0986) (end 145.9636 103.0986) (width 0.6096) (layer "B.Cu") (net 4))
 (segment (start 154.4576 103.0986) (end 154.01935 103.53685) (width 0.8128) (layer "B.Cu") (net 4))
 (segment (start 145.9636 103.0986) (end 145.9611 103.1011) (width 0.6096) (layer "B.Cu") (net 4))
 (segment (start 148.2598 105.41) (end 148.1861 105.4837) (width 0.6096) (layer "B.Cu") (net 6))
 (segment (start 145.9611 105.0011) (end 146.37 105.41) (width 0.6096) (layer "B.Cu") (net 6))
 (segment (start 148.1861 105.4837) (end 148.1861 107.5436) (width 0.6096) (layer "B.Cu") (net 6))
 (segment (start 146.37 105.41) (end 148.2598 105.41) (width 0.6096) (layer "B.Cu") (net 6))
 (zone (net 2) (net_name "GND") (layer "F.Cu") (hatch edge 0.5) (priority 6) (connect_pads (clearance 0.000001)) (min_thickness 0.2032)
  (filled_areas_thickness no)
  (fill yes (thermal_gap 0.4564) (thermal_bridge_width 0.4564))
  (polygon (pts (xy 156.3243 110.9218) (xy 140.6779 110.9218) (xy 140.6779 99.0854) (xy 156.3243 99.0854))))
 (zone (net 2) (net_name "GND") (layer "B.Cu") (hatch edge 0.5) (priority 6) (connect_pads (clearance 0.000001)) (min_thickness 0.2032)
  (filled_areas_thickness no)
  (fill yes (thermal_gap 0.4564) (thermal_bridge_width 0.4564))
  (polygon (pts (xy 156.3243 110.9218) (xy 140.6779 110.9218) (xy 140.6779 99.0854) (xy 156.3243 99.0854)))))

